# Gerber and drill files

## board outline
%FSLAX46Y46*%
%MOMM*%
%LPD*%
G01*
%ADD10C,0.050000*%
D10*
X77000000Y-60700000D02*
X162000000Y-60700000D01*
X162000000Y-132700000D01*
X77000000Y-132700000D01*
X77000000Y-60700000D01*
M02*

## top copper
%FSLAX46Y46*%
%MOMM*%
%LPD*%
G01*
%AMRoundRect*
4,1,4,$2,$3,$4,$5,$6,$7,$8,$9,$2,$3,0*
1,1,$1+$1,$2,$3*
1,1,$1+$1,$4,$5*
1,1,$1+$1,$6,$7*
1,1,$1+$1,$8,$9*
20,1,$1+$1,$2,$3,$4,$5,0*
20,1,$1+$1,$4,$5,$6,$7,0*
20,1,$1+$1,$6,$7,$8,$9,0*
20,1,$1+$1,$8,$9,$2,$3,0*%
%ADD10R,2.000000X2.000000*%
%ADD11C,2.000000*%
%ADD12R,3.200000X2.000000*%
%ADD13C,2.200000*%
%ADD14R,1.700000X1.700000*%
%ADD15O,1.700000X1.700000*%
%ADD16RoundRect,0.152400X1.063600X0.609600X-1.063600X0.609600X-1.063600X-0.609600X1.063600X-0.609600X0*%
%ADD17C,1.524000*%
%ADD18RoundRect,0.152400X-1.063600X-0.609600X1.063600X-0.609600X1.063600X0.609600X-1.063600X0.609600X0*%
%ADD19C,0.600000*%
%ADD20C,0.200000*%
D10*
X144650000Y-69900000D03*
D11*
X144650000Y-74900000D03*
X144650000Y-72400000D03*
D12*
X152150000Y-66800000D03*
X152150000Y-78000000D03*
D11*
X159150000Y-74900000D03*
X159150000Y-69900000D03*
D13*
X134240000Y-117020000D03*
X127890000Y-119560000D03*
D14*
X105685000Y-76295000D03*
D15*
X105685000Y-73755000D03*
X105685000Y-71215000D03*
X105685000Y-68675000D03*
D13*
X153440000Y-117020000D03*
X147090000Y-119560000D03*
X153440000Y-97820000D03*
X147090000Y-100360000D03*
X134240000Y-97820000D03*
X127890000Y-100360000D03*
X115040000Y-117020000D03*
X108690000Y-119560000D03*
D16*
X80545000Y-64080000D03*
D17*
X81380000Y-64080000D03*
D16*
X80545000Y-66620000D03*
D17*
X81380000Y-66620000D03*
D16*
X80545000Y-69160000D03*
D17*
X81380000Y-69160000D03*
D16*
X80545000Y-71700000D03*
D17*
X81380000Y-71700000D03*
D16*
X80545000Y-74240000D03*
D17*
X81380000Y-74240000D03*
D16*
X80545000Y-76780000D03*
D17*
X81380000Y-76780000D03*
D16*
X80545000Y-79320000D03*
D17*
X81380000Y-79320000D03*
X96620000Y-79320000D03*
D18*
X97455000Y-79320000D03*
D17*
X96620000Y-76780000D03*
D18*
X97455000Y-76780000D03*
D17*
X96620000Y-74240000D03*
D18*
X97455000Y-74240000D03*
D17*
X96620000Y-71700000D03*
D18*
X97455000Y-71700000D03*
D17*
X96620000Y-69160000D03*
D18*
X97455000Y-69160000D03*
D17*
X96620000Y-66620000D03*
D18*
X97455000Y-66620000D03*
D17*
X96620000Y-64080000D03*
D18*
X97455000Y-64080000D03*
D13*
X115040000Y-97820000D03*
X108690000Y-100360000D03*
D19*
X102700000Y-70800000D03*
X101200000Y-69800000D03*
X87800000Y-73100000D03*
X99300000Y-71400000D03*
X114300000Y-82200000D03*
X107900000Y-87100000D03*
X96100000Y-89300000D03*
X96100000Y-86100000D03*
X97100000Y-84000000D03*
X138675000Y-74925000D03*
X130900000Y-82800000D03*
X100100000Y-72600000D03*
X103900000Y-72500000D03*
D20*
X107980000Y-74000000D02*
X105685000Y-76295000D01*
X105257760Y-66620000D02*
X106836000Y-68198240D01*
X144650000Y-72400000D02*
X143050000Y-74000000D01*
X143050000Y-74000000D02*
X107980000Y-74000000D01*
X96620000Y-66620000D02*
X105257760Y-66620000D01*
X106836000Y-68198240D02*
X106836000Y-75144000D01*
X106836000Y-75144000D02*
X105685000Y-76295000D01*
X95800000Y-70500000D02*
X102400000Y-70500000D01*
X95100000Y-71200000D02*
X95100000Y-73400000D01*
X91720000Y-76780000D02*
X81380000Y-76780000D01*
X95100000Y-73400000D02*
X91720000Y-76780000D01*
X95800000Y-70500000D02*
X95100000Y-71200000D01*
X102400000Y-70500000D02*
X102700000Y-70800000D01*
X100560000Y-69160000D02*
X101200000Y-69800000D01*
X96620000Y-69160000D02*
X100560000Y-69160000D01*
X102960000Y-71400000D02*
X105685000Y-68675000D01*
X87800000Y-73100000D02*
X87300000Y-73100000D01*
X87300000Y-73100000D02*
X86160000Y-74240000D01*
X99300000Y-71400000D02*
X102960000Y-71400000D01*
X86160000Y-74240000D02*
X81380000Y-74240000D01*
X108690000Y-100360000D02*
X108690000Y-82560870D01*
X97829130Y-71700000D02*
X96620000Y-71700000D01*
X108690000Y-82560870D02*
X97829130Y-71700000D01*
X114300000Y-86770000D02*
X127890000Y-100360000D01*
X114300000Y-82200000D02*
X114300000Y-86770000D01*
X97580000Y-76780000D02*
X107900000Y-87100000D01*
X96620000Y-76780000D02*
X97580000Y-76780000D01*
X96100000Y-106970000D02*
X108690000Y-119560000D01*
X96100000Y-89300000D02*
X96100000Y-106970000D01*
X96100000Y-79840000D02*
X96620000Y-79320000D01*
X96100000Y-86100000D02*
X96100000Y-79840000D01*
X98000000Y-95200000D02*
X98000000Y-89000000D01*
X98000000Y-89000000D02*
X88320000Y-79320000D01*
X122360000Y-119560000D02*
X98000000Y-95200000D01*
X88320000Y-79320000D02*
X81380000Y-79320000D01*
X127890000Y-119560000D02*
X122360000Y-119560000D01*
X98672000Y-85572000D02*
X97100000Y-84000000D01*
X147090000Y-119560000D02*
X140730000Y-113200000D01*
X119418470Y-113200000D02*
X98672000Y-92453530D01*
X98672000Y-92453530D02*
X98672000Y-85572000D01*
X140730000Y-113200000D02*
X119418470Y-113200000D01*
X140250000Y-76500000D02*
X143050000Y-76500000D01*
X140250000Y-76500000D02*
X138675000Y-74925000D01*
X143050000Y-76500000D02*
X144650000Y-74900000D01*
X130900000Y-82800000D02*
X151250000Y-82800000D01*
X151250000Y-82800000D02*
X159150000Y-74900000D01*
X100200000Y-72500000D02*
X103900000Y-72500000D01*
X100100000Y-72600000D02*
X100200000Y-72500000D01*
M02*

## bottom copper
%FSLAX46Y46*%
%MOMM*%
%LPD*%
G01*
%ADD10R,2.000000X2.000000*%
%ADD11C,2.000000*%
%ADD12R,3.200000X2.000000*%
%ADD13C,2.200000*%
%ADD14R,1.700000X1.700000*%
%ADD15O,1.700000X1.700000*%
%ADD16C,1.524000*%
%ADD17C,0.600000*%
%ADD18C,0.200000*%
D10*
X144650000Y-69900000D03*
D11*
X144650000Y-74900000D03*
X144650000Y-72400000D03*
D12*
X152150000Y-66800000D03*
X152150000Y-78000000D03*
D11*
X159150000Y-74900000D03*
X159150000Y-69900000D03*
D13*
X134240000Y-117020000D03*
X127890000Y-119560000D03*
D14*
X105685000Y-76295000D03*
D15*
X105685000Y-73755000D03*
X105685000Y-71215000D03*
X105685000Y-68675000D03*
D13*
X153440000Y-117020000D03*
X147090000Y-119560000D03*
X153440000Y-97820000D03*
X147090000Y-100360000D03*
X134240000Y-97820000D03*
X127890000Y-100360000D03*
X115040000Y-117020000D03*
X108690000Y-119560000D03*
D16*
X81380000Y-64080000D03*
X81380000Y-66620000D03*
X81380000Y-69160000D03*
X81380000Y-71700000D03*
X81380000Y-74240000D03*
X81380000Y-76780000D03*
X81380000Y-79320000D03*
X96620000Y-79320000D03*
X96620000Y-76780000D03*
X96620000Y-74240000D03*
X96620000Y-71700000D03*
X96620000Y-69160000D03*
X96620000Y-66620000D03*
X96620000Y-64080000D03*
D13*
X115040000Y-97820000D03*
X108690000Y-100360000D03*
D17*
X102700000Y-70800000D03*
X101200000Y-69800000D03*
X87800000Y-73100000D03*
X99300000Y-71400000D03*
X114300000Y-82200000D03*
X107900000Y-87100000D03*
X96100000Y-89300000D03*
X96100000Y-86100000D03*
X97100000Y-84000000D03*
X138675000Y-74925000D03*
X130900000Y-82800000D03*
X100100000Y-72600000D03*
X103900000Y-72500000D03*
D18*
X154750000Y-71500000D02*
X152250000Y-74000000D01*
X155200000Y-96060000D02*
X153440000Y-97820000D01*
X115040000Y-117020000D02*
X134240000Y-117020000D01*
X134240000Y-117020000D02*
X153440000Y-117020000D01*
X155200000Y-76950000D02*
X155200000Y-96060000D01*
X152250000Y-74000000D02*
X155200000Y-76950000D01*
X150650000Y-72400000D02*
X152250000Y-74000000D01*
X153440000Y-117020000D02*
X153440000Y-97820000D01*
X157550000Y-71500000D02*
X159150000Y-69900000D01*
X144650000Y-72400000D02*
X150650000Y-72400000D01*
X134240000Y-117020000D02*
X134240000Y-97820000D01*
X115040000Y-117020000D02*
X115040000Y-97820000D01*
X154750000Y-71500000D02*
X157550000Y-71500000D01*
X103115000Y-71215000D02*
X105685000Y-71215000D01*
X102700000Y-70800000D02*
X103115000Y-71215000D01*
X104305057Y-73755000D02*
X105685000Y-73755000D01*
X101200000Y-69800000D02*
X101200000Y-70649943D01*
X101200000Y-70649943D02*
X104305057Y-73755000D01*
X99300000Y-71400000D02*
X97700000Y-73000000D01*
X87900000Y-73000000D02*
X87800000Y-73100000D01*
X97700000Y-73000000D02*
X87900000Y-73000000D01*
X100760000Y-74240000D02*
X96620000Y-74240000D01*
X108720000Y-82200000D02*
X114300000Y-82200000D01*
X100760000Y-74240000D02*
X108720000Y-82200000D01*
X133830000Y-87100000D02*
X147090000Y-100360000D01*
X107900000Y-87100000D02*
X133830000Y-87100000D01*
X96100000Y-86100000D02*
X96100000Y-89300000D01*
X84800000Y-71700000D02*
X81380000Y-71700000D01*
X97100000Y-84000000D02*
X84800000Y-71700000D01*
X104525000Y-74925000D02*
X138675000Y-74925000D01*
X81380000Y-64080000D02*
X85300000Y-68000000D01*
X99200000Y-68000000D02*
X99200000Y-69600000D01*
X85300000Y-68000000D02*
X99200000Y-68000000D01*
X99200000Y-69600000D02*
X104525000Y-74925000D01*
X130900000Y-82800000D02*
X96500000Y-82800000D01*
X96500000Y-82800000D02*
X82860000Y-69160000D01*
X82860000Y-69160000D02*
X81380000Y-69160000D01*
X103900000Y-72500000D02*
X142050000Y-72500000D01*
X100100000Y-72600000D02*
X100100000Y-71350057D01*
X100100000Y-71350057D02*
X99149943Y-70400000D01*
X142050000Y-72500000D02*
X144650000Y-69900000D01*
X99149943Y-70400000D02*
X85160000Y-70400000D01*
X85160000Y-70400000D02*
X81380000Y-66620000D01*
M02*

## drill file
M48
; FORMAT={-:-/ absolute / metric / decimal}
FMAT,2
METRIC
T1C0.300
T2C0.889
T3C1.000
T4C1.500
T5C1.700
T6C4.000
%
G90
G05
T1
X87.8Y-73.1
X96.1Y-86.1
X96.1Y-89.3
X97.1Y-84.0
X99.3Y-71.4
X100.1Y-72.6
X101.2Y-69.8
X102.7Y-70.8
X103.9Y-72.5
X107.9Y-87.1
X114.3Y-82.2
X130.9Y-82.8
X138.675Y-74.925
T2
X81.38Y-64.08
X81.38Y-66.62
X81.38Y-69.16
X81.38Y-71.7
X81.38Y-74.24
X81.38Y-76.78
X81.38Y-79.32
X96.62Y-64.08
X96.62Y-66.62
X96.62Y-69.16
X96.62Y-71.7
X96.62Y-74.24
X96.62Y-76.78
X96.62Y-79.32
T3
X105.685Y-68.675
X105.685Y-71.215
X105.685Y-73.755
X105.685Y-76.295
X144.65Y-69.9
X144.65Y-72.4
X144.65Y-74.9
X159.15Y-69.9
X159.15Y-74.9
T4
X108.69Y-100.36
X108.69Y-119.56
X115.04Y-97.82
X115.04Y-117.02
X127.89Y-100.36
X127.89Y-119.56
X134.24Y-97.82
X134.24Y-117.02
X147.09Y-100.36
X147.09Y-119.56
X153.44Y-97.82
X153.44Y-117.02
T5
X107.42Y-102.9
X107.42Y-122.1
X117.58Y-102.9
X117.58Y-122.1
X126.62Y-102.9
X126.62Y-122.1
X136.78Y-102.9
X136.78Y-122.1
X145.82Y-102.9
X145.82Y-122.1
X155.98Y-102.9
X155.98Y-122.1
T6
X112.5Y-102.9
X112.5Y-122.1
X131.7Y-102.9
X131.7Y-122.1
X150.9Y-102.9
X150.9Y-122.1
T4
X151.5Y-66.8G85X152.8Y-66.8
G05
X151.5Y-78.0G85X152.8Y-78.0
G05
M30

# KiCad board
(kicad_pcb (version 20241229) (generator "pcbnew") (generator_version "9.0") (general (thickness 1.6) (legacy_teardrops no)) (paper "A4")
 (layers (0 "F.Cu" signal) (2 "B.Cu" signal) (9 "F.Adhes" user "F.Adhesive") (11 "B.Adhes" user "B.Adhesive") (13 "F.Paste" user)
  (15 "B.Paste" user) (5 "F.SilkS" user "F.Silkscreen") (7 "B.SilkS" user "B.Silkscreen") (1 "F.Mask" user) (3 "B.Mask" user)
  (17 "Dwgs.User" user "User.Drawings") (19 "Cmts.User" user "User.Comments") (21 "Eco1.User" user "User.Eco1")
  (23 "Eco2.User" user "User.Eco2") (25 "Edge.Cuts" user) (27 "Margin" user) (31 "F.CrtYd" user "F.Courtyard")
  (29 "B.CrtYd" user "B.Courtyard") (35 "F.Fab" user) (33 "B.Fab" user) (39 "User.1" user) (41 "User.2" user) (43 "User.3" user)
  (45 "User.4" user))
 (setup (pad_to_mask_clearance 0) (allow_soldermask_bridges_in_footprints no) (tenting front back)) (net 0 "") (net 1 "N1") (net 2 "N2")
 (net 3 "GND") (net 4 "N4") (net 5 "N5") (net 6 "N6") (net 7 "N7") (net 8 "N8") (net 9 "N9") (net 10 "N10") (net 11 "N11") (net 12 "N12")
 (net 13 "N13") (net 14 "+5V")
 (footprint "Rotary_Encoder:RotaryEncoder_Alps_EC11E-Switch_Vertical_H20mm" (layer "F.Cu") (at 144.65 69.9)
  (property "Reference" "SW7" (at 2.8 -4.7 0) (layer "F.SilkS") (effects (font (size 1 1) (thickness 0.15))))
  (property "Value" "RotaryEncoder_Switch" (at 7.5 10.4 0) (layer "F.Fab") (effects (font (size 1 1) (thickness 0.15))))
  (pad "A" thru_hole rect (at 0 0) (size 2 2) (drill 1) (layers "*.Cu" "*.Mask") (remove_unused_layers no) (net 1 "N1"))
  (pad "B" thru_hole circle (at 0 5) (size 2 2) (drill 1) (layers "*.Cu" "*.Mask") (remove_unused_layers no) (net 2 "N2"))
  (pad "C" thru_hole circle (at 0 2.5) (size 2 2) (drill 1) (layers "*.Cu" "*.Mask") (remove_unused_layers no) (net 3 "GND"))
  (pad "MP" thru_hole rect (at 7.5 -3.1) (size 3.2 2) (drill oval 2.8 1.5) (layers "*.Cu" "*.Mask") (remove_unused_layers no))
  (pad "MP" thru_hole rect (at 7.5 8.1) (size 3.2 2) (drill oval 2.8 1.5) (layers "*.Cu" "*.Mask") (remove_unused_layers no))
  (pad "S1" thru_hole circle (at 14.5 5) (size 2 2) (drill 1) (layers "*.Cu" "*.Mask") (remove_unused_layers no) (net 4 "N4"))
  (pad "S2" thru_hole circle (at 14.5 0) (size 2 2) (drill 1) (layers "*.Cu" "*.Mask") (remove_unused_layers no) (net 3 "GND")))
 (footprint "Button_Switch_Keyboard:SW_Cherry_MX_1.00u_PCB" (layer "F.Cu") (at 134.24 117.02)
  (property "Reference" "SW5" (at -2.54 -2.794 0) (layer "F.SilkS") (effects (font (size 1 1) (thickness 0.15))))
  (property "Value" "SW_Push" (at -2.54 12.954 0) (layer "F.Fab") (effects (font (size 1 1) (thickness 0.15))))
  (pad "" np_thru_hole circle (at -7.62 5.08) (size 1.7 1.7) (drill 1.7) (layers "*.Cu" "*.Mask"))
  (pad "" np_thru_hole circle (at -2.54 5.08) (size 4 4) (drill 4) (layers "*.Cu" "*.Mask"))
  (pad "" np_thru_hole circle (at 2.54 5.08) (size 1.7 1.7) (drill 1.7) (layers "*.Cu" "*.Mask"))
  (pad "1" thru_hole circle (at 0 0) (size 2.2 2.2) (drill 1.5) (layers "*.Cu" "*.Mask") (remove_unused_layers no) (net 3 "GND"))
  (pad "2" thru_hole circle (at -6.35 2.54) (size 2.2 2.2) (drill 1.5) (layers "*.Cu" "*.Mask") (remove_unused_layers no) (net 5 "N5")))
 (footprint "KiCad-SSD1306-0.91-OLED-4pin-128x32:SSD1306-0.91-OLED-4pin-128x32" (layer "F.Cu") (at 142.185 78.485 180)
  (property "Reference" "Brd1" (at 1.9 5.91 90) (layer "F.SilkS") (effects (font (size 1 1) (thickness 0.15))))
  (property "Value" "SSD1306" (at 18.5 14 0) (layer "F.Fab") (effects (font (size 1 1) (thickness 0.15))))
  (pad "1" thru_hole rect (at 36.5 2.19 180) (size 1.7 1.7) (drill 1) (layers "*.Cu" "*.Mask") (remove_unused_layers no) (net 3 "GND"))
  (pad "2" thru_hole oval (at 36.5 4.73 180) (size 1.7 1.7) (drill 1) (layers "*.Cu" "*.Mask") (remove_unused_layers no) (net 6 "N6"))
  (pad "3" thru_hole oval (at 36.5 7.27 180) (size 1.7 1.7) (drill 1) (layers "*.Cu" "*.Mask") (remove_unused_layers no) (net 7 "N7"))
  (pad "4" thru_hole oval (at 36.5 9.81 180) (size 1.7 1.7) (drill 1) (layers "*.Cu" "*.Mask") (remove_unused_layers no) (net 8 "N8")))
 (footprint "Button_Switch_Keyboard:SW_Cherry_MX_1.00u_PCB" (layer "F.Cu") (at 153.44 117.02)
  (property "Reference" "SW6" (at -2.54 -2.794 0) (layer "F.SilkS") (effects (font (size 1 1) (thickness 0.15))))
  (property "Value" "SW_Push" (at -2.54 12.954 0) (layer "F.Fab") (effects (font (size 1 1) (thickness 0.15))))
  (pad "" np_thru_hole circle (at -7.62 5.08) (size 1.7 1.7) (drill 1.7) (layers "*.Cu" "*.Mask"))
  (pad "" np_thru_hole circle (at -2.54 5.08) (size 4 4) (drill 4) (layers "*.Cu" "*.Mask"))
  (pad "" np_thru_hole circle (at 2.54 5.08) (size 1.7 1.7) (drill 1.7) (layers "*.Cu" "*.Mask"))
  (pad "1" thru_hole circle (at 0 0) (size 2.2 2.2) (drill 1.5) (layers "*.Cu" "*.Mask") (remove_unused_layers no) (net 3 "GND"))
  (pad "2" thru_hole circle (at -6.35 2.54) (size 2.2 2.2) (drill 1.5) (layers "*.Cu" "*.Mask") (remove_unused_layers no) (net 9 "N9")))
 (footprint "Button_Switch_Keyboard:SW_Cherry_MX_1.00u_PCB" (layer "F.Cu") (at 153.44 97.82)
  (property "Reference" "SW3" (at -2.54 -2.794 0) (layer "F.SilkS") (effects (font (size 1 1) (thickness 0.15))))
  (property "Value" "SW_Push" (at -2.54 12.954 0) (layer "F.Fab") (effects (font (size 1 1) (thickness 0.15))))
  (pad "" np_thru_hole circle (at -7.62 5.08) (size 1.7 1.7) (drill 1.7) (layers "*.Cu" "*.Mask"))
  (pad "" np_thru_hole circle (at -2.54 5.08) (size 4 4) (drill 4) (layers "*.Cu" "*.Mask"))
  (pad "" np_thru_hole circle (at 2.54 5.08) (size 1.7 1.7) (drill 1.7) (layers "*.Cu" "*.Mask"))
  (pad "1" thru_hole circle (at 0 0) (size 2.2 2.2) (drill 1.5) (layers "*.Cu" "*.Mask") (remove_unused_layers no) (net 3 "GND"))
  (pad "2" thru_hole circle (at -6.35 2.54) (size 2.2 2.2) (drill 1.5) (layers "*.Cu" "*.Mask") (remove_unused_layers no) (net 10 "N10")))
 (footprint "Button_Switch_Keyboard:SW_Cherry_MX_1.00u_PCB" (layer "F.Cu") (at 134.24 97.82)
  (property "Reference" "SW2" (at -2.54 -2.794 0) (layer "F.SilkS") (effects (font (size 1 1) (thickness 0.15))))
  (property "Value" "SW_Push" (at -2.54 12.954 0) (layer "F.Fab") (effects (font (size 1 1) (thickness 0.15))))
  (pad "" np_thru_hole circle (at -7.62 5.08) (size 1.7 1.7) (drill 1.7) (layers "*.Cu" "*.Mask"))
  (pad "" np_thru_hole circle (at -2.54 5.08) (size 4 4) (drill 4) (layers "*.Cu" "*.Mask"))
  (pad "" np_thru_hole circle (at 2.54 5.08) (size 1.7 1.7) (drill 1.7) (layers "*.Cu" "*.Mask"))
  (pad "1" thru_hole circle (at 0 0) (size 2.2 2.2) (drill 1.5) (layers "*.Cu" "*.Mask") (remove_unused_layers no) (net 3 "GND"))
  (pad "2" thru_hole circle (at -6.35 2.54) (size 2.2 2.2) (drill 1.5) (layers "*.Cu" "*.Mask") (remove_unused_layers no) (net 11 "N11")))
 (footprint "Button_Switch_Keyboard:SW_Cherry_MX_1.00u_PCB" (layer "F.Cu") (at 115.04 117.02)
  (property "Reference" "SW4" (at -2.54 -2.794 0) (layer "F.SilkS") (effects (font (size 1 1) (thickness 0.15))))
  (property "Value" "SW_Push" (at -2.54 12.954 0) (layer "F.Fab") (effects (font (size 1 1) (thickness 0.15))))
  (pad "" np_thru_hole circle (at -7.62 5.08) (size 1.7 1.7) (drill 1.7) (layers "*.Cu" "*.Mask"))
  (pad "" np_thru_hole circle (at -2.54 5.08) (size 4 4) (drill 4) (layers "*.Cu" "*.Mask"))
  (pad "" np_thru_hole circle (at 2.54 5.08) (size 1.7 1.7) (drill 1.7) (layers "*.Cu" "*.Mask"))
  (pad "1" thru_hole circle (at 0 0) (size 2.2 2.2) (drill 1.5) (layers "*.Cu" "*.Mask") (remove_unused_layers no) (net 3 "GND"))
  (pad "2" thru_hole circle (at -6.35 2.54) (size 2.2 2.2) (drill 1.5) (layers "*.Cu" "*.Mask") (remove_unused_layers no) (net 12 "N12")))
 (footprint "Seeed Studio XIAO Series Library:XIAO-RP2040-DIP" (layer "F.Cu") (at 89 71.7)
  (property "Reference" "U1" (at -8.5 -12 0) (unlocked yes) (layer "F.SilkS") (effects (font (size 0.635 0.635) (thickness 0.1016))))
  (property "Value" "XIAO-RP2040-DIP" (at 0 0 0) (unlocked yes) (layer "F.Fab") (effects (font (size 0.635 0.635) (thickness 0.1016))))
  (pad "1" smd roundrect (at -8.455 -7.62 180) (size 2.432 1.524) (layers "F.Cu" "F.Mask") (roundrect_rratio 0.1) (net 2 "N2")
   (thermal_bridge_angle 45))
  (pad "1" thru_hole circle (at -7.62 -7.62 180) (size 1.524 1.524) (drill 0.889) (layers "*.Cu" "*.Mask") (remove_unused_layers no)
   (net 2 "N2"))
  (pad "2" smd roundrect (at -8.455 -5.08 180) (size 2.432 1.524) (layers "F.Cu" "F.Mask") (roundrect_rratio 0.1) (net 1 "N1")
   (thermal_bridge_angle 45))
  (pad "2" thru_hole circle (at -7.62 -5.08 180) (size 1.524 1.524) (drill 0.889) (layers "*.Cu" "*.Mask") (remove_unused_layers no)
   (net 1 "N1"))
  (pad "3" smd roundrect (at -8.455 -2.54 180) (size 2.432 1.524) (layers "F.Cu" "F.Mask") (roundrect_rratio 0.1) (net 4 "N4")
   (thermal_bridge_angle 45))
  (pad "3" thru_hole circle (at -7.62 -2.54 180) (size 1.524 1.524) (drill 0.889) (layers "*.Cu" "*.Mask") (remove_unused_layers no)
   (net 4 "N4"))
  (pad "4" smd roundrect (at -8.455 0 180) (size 2.432 1.524) (layers "F.Cu" "F.Mask") (roundrect_rratio 0.1) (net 9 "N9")
   (thermal_bridge_angle 45))
  (pad "4" thru_hole circle (at -7.62 0 180) (size 1.524 1.524) (drill 0.889) (layers "*.Cu" "*.Mask") (remove_unused_layers no)
   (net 9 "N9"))
  (pad "5" smd roundrect (at -8.455 2.54 180) (size 2.432 1.524) (layers "F.Cu" "F.Mask") (roundrect_rratio 0.1) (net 8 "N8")
   (thermal_bridge_angle 45))
  (pad "5" thru_hole circle (at -7.62 2.54 180) (size 1.524 1.524) (drill 0.889) (layers "*.Cu" "*.Mask") (remove_unused_layers no)
   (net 8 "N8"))
  (pad "6" smd roundrect (at -8.455 5.08 180) (size 2.432 1.524) (layers "F.Cu" "F.Mask") (roundrect_rratio 0.1) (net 7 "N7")
   (thermal_bridge_angle 45))
  (pad "6" thru_hole circle (at -7.62 5.08 180) (size 1.524 1.524) (drill 0.889) (layers "*.Cu" "*.Mask") (remove_unused_layers no)
   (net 7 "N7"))
  (pad "7" smd roundrect (at -8.455 7.62 180) (size 2.432 1.524) (layers "F.Cu" "F.Mask") (roundrect_rratio 0.1) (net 5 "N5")
   (thermal_bridge_angle 45))
  (pad "7" thru_hole circle (at -7.62 7.62 180) (size 1.524 1.524) (drill 0.889) (layers "*.Cu" "*.Mask") (remove_unused_layers no)
   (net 5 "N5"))
  (pad "8" thru_hole circle (at 7.62 7.62) (size 1.524 1.524) (drill 0.889) (layers "*.Cu" "*.Mask") (remove_unused_layers no)
   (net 12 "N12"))
  (pad "8" smd roundrect (at 8.455 7.62) (size 2.432 1.524) (layers "F.Cu" "F.Mask") (roundrect_rratio 0.1) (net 12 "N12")
   (thermal_bridge_angle 45))
  (pad "9" thru_hole circle (at 7.62 5.08) (size 1.524 1.524) (drill 0.889) (layers "*.Cu" "*.Mask") (remove_unused_layers no)
   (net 10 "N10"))
  (pad "9" smd roundrect (at 8.455 5.08) (size 2.432 1.524) (layers "F.Cu" "F.Mask") (roundrect_rratio 0.1) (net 10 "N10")
   (thermal_bridge_angle 45))
  (pad "10" thru_hole circle (at 7.62 2.54) (size 1.524 1.524) (drill 0.889) (layers "*.Cu" "*.Mask") (remove_unused_layers no)
   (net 11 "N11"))
  (pad "10" smd roundrect (at 8.455 2.54) (size 2.432 1.524) (layers "F.Cu" "F.Mask") (roundrect_rratio 0.1) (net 11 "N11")
   (thermal_bridge_angle 45))
  (pad "11" thru_hole circle (at 7.62 0) (size 1.524 1.524) (drill 0.889) (layers "*.Cu" "*.Mask") (remove_unused_layers no) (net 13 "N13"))
  (pad "11" smd roundrect (at 8.455 0) (size 2.432 1.524) (layers "F.Cu" "F.Mask") (roundrect_rratio 0.1) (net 13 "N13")
   (thermal_bridge_angle 45))
  (pad "12" thru_hole circle (at 7.62 -2.54) (size 1.524 1.524) (drill 0.889) (layers "*.Cu" "*.Mask") (remove_unused_layers no)
   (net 6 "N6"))
  (pad "12" smd roundrect (at 8.455 -2.54) (size 2.432 1.524) (layers "F.Cu" "F.Mask") (roundrect_rratio 0.1) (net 6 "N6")
   (thermal_bridge_angle 45))
  (pad "13" thru_hole circle (at 7.62 -5.08) (size 1.524 1.524) (drill 0.889) (layers "*.Cu" "*.Mask") (remove_unused_layers no)
   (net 3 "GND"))
  (pad "13" smd roundrect (at 8.455 -5.08) (size 2.432 1.524) (layers "F.Cu" "F.Mask") (roundrect_rratio 0.1) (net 3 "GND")
   (thermal_bridge_angle 45))
  (pad "14" thru_hole circle (at 7.62 -7.62) (size 1.524 1.524) (drill 0.889) (layers "*.Cu" "*.Mask") (remove_unused_layers no)
   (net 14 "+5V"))
  (pad "14" smd roundrect (at 8.455 -7.62) (size 2.432 1.524) (layers "F.Cu" "F.Mask") (roundrect_rratio 0.1) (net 14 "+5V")
   (thermal_bridge_angle 45)))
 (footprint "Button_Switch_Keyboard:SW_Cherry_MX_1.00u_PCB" (layer "F.Cu") (at 115.04 97.82)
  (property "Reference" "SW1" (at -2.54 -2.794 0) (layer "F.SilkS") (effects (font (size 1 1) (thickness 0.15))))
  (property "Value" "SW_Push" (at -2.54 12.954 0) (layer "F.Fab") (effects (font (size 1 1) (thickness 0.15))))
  (pad "" np_thru_hole circle (at -7.62 5.08) (size 1.7 1.7) (drill 1.7) (layers "*.Cu" "*.Mask"))
  (pad "" np_thru_hole circle (at -2.54 5.08) (size 4 4) (drill 4) (layers "*.Cu" "*.Mask"))
  (pad "" np_thru_hole circle (at 2.54 5.08) (size 1.7 1.7) (drill 1.7) (layers "*.Cu" "*.Mask"))
  (pad "1" thru_hole circle (at 0 0) (size 2.2 2.2) (drill 1.5) (layers "*.Cu" "*.Mask") (remove_unused_layers no) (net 3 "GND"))
  (pad "2" thru_hole circle (at -6.35 2.54) (size 2.2 2.2) (drill 1.5) (layers "*.Cu" "*.Mask") (remove_unused_layers no) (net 13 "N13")))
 (gr_rect (start 77 60.7) (end 162 132.7) (stroke (width 0.05) (type default)) (fill no) (layer "Edge.Cuts"))
 (segment (start 107.98 74) (end 105.685 76.295) (width 0.2) (layer "F.Cu") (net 3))
 (segment (start 105.25776 66.62) (end 106.836 68.19824) (width 0.2) (layer "F.Cu") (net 3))
 (segment (start 144.65 72.4) (end 143.05 74) (width 0.2) (layer "F.Cu") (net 3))
 (segment (start 143.05 74) (end 107.98 74) (width 0.2) (layer "F.Cu") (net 3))
 (segment (start 96.62 66.62) (end 105.25776 66.62) (width 0.2) (layer "F.Cu") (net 3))
 (segment (start 106.836 68.19824) (end 106.836 75.144) (width 0.2) (layer "F.Cu") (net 3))
 (segment (start 106.836 75.144) (end 105.685 76.295) (width 0.2) (layer "F.Cu") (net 3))
 (segment (start 154.75 71.5) (end 152.25 74) (width 0.2) (layer "B.Cu") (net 3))
 (segment (start 155.2 96.06) (end 153.44 97.82) (width 0.2) (layer "B.Cu") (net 3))
 (segment (start 115.04 117.02) (end 134.24 117.02) (width 0.2) (layer "B.Cu") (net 3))
 (segment (start 134.24 117.02) (end 153.44 117.02) (width 0.2) (layer "B.Cu") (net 3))
 (segment (start 155.2 76.95) (end 155.2 96.06) (width 0.2) (layer "B.Cu") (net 3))
 (segment (start 152.25 74) (end 155.2 76.95) (width 0.2) (layer "B.Cu") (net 3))
 (segment (start 150.65 72.4) (end 152.25 74) (width 0.2) (layer "B.Cu") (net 3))
 (segment (start 153.44 117.02) (end 153.44 97.82) (width 0.2) (layer "B.Cu") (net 3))
 (segment (start 157.55 71.5) (end 159.15 69.9) (width 0.2) (layer "B.Cu") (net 3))
 (segment (start 144.65 72.4) (end 150.65 72.4) (width 0.2) (layer "B.Cu") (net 3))
 (segment (start 134.24 117.02) (end 134.24 97.82) (width 0.2) (layer "B.Cu") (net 3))
 (segment (start 115.04 117.02) (end 115.04 97.82) (width 0.2) (layer "B.Cu") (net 3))
 (segment (start 154.75 71.5) (end 157.55 71.5) (width 0.2) (layer "B.Cu") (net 3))
 (segment (start 95.8 70.5) (end 102.4 70.5) (width 0.2) (layer "F.Cu") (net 7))
 (segment (start 95.1 71.2) (end 95.1 73.4) (width 0.2) (layer "F.Cu") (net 7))
 (segment (start 91.72 76.78) (end 81.38 76.78) (width 0.2) (layer "F.Cu") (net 7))
 (segment (start 95.1 73.4) (end 91.72 76.78) (width 0.2) (layer "F.Cu") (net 7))
 (segment (start 95.8 70.5) (end 95.1 71.2) (width 0.2) (layer "F.Cu") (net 7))
 (segment (start 102.4 70.5) (end 102.7 70.8) (width 0.2) (layer "F.Cu") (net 7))
 (via (at 102.7 70.8) (size 0.6) (drill 0.3) (layers "F.Cu" "B.Cu") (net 7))
 (segment (start 103.115 71.215) (end 105.685 71.215) (width 0.2) (layer "B.Cu") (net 7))
 (segment (start 102.7 70.8) (end 103.115 71.215) (width 0.2) (layer "B.Cu") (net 7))
 (segment (start 100.56 69.16) (end 101.2 69.8) (width 0.2) (layer "F.Cu") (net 6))
 (segment (start 96.62 69.16) (end 100.56 69.16) (width 0.2) (layer "F.Cu") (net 6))
 (via (at 101.2 69.8) (size 0.6) (drill 0.3) (layers "F.Cu" "B.Cu") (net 6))
 (segment (start 104.305057 73.755) (end 105.685 73.755) (width 0.2) (layer "B.Cu") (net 6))
 (segment (start 101.2 69.8) (end 101.2 70.649943) (width 0.2) (layer "B.Cu") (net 6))
 (segment (start 101.2 70.649943) (end 104.305057 73.755) (width 0.2) (layer "B.Cu") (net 6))
 (segment (start 102.96 71.4) (end 105.685 68.675) (width 0.2) (layer "F.Cu") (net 8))
 (segment (start 87.8 73.1) (end 87.3 73.1) (width 0.2) (layer "F.Cu") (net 8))
 (segment (start 87.3 73.1) (end 86.16 74.24) (width 0.2) (layer "F.Cu") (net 8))
 (segment (start 99.3 71.4) (end 102.96 71.4) (width 0.2) (layer "F.Cu") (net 8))
 (segment (start 86.16 74.24) (end 81.38 74.24) (width 0.2) (layer "F.Cu") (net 8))
 (via (at 87.8 73.1) (size 0.6) (drill 0.3) (layers "F.Cu" "B.Cu") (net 8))
 (via (at 99.3 71.4) (size 0.6) (drill 0.3) (layers "F.Cu" "B.Cu") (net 8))
 (segment (start 99.3 71.4) (end 97.7 73) (width 0.2) (layer "B.Cu") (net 8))
 (segment (start 87.9 73) (end 87.8 73.1) (width 0.2) (layer "B.Cu") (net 8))
 (segment (start 97.7 73) (end 87.9 73) (width 0.2) (layer "B.Cu") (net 8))
 (segment (start 108.69 100.36) (end 108.69 82.56087) (width 0.2) (layer "F.Cu") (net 13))
 (segment (start 97.82913 71.7) (end 96.62 71.7) (width 0.2) (layer "F.Cu") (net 13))
 (segment (start 108.69 82.56087) (end 97.82913 71.7) (width 0.2) (layer "F.Cu") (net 13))
 (segment (start 114.3 86.77) (end 127.89 100.36) (width 0.2) (layer "F.Cu") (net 11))
 (segment (start 114.3 82.2) (end 114.3 86.77) (width 0.2) (layer "F.Cu") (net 11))
 (via (at 114.3 82.2) (size 0.6) (drill 0.3) (layers "F.Cu" "B.Cu") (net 11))
 (segment (start 100.76 74.24) (end 96.62 74.24) (width 0.2) (layer "B.Cu") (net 11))
 (segment (start 108.72 82.2) (end 114.3 82.2) (width 0.2) (layer "B.Cu") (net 11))
 (segment (start 100.76 74.24) (end 108.72 82.2) (width 0.2) (layer "B.Cu") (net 11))
 (segment (start 97.58 76.78) (end 107.9 87.1) (width 0.2) (layer "F.Cu") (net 10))
 (segment (start 96.62 76.78) (end 97.58 76.78) (width 0.2) (layer "F.Cu") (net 10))
 (via (at 107.9 87.1) (size 0.6) (drill 0.3) (layers "F.Cu" "B.Cu") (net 10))
 (segment (start 133.83 87.1) (end 147.09 100.36) (width 0.2) (layer "B.Cu") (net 10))
 (segment (start 107.9 87.1) (end 133.83 87.1) (width 0.2) (layer "B.Cu") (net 10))
 (segment (start 96.1 106.97) (end 108.69 119.56) (width 0.2) (layer "F.Cu") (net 12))
 (segment (start 96.1 89.3) (end 96.1 106.97) (width 0.2) (layer "F.Cu") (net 12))
 (segment (start 96.1 79.84) (end 96.62 79.32) (width 0.2) (layer "F.Cu") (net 12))
 (segment (start 96.1 86.1) (end 96.1 79.84) (width 0.2) (layer "F.Cu") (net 12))
 (via (at 96.1 89.3) (size 0.6) (drill 0.3) (layers "F.Cu" "B.Cu") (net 12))
 (via (at 96.1 86.1) (size 0.6) (drill 0.3) (layers "F.Cu" "B.Cu") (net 12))
 (segment (start 96.1 86.1) (end 96.1 89.3) (width 0.2) (layer "B.Cu") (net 12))
 (segment (start 98 95.2) (end 98 89) (width 0.2) (layer "F.Cu") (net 5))
 (segment (start 98 89) (end 88.32 79.32) (width 0.2) (layer "F.Cu") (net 5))
 (segment (start 122.36 119.56) (end 98 95.2) (width 0.2) (layer "F.Cu") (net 5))
 (segment (start 88.32 79.32) (end 81.38 79.32) (width 0.2) (layer "F.Cu") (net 5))
 (segment (start 127.89 119.56) (end 122.36 119.56) (width 0.2) (layer "F.Cu") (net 5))
 (segment (start 98.672 85.572) (end 97.1 84) (width 0.2) (layer "F.Cu") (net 9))
 (segment (start 147.09 119.56) (end 140.73 113.2) (width 0.2) (layer "F.Cu") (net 9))
 (segment (start 119.41847 113.2) (end 98.672 92.45353) (width 0.2) (layer "F.Cu") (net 9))
 (segment (start 98.672 92.45353) (end 98.672 85.572) (width 0.2) (layer "F.Cu") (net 9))
 (segment (start 140.73 113.2) (end 119.41847 113.2) (width 0.2) (layer "F.Cu") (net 9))
 (via (at 97.1 84) (size 0.6) (drill 0.3) (layers "F.Cu" "B.Cu") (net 9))
 (segment (start 84.8 71.7) (end 81.38 71.7) (width 0.2) (layer "B.Cu") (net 9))
 (segment (start 97.1 84) (end 84.8 71.7) (width 0.2) (layer "B.Cu") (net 9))
 (segment (start 140.25 76.5) (end 143.05 76.5) (width 0.2) (layer "F.Cu") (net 2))
 (segment (start 140.25 76.5) (end 138.675 74.925) (width 0.2) (layer "F.Cu") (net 2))
 (segment (start 143.05 76.5) (end 144.65 74.9) (width 0.2) (layer "F.Cu") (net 2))
 (via (at 138.675 74.925) (size 0.6) (drill 0.3) (layers "F.Cu" "B.Cu") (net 2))
 (segment (start 104.525 74.925) (end 138.675 74.925) (width 0.2) (layer "B.Cu") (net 2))
 (segment (start 81.38 64.08) (end 85.3 68) (width 0.2) (layer "B.Cu") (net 2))
 (segment (start 99.2 68) (end 99.2 69.6) (width 0.2) (layer "B.Cu") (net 2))
 (segment (start 85.3 68) (end 99.2 68) (width 0.2) (layer "B.Cu") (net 2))
 (segment (start 99.2 69.6) (end 104.525 74.925) (width 0.2) (layer "B.Cu") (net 2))
 (segment (start 130.9 82.8) (end 151.25 82.8) (width 0.2) (layer "F.Cu") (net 4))
 (segment (start 151.25 82.8) (end 159.15 74.9) (width 0.2) (layer "F.Cu") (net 4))
 (via (at 130.9 82.8) (size 0.6) (drill 0.3) (layers "F.Cu" "B.Cu") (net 4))
 (segment (start 130.9 82.8) (end 96.5 82.8) (width 0.2) (layer "B.Cu") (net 4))
 (segment (start 96.5 82.8) (end 82.86 69.16) (width 0.2) (layer "B.Cu") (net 4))
 (segment (start 82.86 69.16) (end 81.38 69.16) (width 0.2) (layer "B.Cu") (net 4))
 (segment (start 100.2 72.5) (end 103.9 72.5) (width 0.2) (layer "F.Cu") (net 1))
 (segment (start 100.1 72.6) (end 100.2 72.5) (width 0.2) (layer "F.Cu") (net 1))
 (via (at 100.1 72.6) (size 0.6) (drill 0.3) (layers "F.Cu" "B.Cu") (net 1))
 (via (at 103.9 72.5) (size 0.6) (drill 0.3) (layers "F.Cu" "B.Cu") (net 1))
 (segment (start 103.9 72.5) (end 142.05 72.5) (width 0.2) (layer "B.Cu") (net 1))
 (segment (start 100.1 72.6) (end 100.1 71.350057) (width 0.2) (layer "B.Cu") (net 1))
 (segment (start 100.1 71.350057) (end 99.149943 70.4) (width 0.2) (layer "B.Cu") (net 1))
 (segment (start 142.05 72.5) (end 144.65 69.9) (width 0.2) (layer "B.Cu") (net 1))
 (segment (start 99.149943 70.4) (end 85.16 70.4) (width 0.2) (layer "B.Cu") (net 1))
 (segment (start 85.16 70.4) (end 81.38 66.62) (width 0.2) (layer "B.Cu") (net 1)))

